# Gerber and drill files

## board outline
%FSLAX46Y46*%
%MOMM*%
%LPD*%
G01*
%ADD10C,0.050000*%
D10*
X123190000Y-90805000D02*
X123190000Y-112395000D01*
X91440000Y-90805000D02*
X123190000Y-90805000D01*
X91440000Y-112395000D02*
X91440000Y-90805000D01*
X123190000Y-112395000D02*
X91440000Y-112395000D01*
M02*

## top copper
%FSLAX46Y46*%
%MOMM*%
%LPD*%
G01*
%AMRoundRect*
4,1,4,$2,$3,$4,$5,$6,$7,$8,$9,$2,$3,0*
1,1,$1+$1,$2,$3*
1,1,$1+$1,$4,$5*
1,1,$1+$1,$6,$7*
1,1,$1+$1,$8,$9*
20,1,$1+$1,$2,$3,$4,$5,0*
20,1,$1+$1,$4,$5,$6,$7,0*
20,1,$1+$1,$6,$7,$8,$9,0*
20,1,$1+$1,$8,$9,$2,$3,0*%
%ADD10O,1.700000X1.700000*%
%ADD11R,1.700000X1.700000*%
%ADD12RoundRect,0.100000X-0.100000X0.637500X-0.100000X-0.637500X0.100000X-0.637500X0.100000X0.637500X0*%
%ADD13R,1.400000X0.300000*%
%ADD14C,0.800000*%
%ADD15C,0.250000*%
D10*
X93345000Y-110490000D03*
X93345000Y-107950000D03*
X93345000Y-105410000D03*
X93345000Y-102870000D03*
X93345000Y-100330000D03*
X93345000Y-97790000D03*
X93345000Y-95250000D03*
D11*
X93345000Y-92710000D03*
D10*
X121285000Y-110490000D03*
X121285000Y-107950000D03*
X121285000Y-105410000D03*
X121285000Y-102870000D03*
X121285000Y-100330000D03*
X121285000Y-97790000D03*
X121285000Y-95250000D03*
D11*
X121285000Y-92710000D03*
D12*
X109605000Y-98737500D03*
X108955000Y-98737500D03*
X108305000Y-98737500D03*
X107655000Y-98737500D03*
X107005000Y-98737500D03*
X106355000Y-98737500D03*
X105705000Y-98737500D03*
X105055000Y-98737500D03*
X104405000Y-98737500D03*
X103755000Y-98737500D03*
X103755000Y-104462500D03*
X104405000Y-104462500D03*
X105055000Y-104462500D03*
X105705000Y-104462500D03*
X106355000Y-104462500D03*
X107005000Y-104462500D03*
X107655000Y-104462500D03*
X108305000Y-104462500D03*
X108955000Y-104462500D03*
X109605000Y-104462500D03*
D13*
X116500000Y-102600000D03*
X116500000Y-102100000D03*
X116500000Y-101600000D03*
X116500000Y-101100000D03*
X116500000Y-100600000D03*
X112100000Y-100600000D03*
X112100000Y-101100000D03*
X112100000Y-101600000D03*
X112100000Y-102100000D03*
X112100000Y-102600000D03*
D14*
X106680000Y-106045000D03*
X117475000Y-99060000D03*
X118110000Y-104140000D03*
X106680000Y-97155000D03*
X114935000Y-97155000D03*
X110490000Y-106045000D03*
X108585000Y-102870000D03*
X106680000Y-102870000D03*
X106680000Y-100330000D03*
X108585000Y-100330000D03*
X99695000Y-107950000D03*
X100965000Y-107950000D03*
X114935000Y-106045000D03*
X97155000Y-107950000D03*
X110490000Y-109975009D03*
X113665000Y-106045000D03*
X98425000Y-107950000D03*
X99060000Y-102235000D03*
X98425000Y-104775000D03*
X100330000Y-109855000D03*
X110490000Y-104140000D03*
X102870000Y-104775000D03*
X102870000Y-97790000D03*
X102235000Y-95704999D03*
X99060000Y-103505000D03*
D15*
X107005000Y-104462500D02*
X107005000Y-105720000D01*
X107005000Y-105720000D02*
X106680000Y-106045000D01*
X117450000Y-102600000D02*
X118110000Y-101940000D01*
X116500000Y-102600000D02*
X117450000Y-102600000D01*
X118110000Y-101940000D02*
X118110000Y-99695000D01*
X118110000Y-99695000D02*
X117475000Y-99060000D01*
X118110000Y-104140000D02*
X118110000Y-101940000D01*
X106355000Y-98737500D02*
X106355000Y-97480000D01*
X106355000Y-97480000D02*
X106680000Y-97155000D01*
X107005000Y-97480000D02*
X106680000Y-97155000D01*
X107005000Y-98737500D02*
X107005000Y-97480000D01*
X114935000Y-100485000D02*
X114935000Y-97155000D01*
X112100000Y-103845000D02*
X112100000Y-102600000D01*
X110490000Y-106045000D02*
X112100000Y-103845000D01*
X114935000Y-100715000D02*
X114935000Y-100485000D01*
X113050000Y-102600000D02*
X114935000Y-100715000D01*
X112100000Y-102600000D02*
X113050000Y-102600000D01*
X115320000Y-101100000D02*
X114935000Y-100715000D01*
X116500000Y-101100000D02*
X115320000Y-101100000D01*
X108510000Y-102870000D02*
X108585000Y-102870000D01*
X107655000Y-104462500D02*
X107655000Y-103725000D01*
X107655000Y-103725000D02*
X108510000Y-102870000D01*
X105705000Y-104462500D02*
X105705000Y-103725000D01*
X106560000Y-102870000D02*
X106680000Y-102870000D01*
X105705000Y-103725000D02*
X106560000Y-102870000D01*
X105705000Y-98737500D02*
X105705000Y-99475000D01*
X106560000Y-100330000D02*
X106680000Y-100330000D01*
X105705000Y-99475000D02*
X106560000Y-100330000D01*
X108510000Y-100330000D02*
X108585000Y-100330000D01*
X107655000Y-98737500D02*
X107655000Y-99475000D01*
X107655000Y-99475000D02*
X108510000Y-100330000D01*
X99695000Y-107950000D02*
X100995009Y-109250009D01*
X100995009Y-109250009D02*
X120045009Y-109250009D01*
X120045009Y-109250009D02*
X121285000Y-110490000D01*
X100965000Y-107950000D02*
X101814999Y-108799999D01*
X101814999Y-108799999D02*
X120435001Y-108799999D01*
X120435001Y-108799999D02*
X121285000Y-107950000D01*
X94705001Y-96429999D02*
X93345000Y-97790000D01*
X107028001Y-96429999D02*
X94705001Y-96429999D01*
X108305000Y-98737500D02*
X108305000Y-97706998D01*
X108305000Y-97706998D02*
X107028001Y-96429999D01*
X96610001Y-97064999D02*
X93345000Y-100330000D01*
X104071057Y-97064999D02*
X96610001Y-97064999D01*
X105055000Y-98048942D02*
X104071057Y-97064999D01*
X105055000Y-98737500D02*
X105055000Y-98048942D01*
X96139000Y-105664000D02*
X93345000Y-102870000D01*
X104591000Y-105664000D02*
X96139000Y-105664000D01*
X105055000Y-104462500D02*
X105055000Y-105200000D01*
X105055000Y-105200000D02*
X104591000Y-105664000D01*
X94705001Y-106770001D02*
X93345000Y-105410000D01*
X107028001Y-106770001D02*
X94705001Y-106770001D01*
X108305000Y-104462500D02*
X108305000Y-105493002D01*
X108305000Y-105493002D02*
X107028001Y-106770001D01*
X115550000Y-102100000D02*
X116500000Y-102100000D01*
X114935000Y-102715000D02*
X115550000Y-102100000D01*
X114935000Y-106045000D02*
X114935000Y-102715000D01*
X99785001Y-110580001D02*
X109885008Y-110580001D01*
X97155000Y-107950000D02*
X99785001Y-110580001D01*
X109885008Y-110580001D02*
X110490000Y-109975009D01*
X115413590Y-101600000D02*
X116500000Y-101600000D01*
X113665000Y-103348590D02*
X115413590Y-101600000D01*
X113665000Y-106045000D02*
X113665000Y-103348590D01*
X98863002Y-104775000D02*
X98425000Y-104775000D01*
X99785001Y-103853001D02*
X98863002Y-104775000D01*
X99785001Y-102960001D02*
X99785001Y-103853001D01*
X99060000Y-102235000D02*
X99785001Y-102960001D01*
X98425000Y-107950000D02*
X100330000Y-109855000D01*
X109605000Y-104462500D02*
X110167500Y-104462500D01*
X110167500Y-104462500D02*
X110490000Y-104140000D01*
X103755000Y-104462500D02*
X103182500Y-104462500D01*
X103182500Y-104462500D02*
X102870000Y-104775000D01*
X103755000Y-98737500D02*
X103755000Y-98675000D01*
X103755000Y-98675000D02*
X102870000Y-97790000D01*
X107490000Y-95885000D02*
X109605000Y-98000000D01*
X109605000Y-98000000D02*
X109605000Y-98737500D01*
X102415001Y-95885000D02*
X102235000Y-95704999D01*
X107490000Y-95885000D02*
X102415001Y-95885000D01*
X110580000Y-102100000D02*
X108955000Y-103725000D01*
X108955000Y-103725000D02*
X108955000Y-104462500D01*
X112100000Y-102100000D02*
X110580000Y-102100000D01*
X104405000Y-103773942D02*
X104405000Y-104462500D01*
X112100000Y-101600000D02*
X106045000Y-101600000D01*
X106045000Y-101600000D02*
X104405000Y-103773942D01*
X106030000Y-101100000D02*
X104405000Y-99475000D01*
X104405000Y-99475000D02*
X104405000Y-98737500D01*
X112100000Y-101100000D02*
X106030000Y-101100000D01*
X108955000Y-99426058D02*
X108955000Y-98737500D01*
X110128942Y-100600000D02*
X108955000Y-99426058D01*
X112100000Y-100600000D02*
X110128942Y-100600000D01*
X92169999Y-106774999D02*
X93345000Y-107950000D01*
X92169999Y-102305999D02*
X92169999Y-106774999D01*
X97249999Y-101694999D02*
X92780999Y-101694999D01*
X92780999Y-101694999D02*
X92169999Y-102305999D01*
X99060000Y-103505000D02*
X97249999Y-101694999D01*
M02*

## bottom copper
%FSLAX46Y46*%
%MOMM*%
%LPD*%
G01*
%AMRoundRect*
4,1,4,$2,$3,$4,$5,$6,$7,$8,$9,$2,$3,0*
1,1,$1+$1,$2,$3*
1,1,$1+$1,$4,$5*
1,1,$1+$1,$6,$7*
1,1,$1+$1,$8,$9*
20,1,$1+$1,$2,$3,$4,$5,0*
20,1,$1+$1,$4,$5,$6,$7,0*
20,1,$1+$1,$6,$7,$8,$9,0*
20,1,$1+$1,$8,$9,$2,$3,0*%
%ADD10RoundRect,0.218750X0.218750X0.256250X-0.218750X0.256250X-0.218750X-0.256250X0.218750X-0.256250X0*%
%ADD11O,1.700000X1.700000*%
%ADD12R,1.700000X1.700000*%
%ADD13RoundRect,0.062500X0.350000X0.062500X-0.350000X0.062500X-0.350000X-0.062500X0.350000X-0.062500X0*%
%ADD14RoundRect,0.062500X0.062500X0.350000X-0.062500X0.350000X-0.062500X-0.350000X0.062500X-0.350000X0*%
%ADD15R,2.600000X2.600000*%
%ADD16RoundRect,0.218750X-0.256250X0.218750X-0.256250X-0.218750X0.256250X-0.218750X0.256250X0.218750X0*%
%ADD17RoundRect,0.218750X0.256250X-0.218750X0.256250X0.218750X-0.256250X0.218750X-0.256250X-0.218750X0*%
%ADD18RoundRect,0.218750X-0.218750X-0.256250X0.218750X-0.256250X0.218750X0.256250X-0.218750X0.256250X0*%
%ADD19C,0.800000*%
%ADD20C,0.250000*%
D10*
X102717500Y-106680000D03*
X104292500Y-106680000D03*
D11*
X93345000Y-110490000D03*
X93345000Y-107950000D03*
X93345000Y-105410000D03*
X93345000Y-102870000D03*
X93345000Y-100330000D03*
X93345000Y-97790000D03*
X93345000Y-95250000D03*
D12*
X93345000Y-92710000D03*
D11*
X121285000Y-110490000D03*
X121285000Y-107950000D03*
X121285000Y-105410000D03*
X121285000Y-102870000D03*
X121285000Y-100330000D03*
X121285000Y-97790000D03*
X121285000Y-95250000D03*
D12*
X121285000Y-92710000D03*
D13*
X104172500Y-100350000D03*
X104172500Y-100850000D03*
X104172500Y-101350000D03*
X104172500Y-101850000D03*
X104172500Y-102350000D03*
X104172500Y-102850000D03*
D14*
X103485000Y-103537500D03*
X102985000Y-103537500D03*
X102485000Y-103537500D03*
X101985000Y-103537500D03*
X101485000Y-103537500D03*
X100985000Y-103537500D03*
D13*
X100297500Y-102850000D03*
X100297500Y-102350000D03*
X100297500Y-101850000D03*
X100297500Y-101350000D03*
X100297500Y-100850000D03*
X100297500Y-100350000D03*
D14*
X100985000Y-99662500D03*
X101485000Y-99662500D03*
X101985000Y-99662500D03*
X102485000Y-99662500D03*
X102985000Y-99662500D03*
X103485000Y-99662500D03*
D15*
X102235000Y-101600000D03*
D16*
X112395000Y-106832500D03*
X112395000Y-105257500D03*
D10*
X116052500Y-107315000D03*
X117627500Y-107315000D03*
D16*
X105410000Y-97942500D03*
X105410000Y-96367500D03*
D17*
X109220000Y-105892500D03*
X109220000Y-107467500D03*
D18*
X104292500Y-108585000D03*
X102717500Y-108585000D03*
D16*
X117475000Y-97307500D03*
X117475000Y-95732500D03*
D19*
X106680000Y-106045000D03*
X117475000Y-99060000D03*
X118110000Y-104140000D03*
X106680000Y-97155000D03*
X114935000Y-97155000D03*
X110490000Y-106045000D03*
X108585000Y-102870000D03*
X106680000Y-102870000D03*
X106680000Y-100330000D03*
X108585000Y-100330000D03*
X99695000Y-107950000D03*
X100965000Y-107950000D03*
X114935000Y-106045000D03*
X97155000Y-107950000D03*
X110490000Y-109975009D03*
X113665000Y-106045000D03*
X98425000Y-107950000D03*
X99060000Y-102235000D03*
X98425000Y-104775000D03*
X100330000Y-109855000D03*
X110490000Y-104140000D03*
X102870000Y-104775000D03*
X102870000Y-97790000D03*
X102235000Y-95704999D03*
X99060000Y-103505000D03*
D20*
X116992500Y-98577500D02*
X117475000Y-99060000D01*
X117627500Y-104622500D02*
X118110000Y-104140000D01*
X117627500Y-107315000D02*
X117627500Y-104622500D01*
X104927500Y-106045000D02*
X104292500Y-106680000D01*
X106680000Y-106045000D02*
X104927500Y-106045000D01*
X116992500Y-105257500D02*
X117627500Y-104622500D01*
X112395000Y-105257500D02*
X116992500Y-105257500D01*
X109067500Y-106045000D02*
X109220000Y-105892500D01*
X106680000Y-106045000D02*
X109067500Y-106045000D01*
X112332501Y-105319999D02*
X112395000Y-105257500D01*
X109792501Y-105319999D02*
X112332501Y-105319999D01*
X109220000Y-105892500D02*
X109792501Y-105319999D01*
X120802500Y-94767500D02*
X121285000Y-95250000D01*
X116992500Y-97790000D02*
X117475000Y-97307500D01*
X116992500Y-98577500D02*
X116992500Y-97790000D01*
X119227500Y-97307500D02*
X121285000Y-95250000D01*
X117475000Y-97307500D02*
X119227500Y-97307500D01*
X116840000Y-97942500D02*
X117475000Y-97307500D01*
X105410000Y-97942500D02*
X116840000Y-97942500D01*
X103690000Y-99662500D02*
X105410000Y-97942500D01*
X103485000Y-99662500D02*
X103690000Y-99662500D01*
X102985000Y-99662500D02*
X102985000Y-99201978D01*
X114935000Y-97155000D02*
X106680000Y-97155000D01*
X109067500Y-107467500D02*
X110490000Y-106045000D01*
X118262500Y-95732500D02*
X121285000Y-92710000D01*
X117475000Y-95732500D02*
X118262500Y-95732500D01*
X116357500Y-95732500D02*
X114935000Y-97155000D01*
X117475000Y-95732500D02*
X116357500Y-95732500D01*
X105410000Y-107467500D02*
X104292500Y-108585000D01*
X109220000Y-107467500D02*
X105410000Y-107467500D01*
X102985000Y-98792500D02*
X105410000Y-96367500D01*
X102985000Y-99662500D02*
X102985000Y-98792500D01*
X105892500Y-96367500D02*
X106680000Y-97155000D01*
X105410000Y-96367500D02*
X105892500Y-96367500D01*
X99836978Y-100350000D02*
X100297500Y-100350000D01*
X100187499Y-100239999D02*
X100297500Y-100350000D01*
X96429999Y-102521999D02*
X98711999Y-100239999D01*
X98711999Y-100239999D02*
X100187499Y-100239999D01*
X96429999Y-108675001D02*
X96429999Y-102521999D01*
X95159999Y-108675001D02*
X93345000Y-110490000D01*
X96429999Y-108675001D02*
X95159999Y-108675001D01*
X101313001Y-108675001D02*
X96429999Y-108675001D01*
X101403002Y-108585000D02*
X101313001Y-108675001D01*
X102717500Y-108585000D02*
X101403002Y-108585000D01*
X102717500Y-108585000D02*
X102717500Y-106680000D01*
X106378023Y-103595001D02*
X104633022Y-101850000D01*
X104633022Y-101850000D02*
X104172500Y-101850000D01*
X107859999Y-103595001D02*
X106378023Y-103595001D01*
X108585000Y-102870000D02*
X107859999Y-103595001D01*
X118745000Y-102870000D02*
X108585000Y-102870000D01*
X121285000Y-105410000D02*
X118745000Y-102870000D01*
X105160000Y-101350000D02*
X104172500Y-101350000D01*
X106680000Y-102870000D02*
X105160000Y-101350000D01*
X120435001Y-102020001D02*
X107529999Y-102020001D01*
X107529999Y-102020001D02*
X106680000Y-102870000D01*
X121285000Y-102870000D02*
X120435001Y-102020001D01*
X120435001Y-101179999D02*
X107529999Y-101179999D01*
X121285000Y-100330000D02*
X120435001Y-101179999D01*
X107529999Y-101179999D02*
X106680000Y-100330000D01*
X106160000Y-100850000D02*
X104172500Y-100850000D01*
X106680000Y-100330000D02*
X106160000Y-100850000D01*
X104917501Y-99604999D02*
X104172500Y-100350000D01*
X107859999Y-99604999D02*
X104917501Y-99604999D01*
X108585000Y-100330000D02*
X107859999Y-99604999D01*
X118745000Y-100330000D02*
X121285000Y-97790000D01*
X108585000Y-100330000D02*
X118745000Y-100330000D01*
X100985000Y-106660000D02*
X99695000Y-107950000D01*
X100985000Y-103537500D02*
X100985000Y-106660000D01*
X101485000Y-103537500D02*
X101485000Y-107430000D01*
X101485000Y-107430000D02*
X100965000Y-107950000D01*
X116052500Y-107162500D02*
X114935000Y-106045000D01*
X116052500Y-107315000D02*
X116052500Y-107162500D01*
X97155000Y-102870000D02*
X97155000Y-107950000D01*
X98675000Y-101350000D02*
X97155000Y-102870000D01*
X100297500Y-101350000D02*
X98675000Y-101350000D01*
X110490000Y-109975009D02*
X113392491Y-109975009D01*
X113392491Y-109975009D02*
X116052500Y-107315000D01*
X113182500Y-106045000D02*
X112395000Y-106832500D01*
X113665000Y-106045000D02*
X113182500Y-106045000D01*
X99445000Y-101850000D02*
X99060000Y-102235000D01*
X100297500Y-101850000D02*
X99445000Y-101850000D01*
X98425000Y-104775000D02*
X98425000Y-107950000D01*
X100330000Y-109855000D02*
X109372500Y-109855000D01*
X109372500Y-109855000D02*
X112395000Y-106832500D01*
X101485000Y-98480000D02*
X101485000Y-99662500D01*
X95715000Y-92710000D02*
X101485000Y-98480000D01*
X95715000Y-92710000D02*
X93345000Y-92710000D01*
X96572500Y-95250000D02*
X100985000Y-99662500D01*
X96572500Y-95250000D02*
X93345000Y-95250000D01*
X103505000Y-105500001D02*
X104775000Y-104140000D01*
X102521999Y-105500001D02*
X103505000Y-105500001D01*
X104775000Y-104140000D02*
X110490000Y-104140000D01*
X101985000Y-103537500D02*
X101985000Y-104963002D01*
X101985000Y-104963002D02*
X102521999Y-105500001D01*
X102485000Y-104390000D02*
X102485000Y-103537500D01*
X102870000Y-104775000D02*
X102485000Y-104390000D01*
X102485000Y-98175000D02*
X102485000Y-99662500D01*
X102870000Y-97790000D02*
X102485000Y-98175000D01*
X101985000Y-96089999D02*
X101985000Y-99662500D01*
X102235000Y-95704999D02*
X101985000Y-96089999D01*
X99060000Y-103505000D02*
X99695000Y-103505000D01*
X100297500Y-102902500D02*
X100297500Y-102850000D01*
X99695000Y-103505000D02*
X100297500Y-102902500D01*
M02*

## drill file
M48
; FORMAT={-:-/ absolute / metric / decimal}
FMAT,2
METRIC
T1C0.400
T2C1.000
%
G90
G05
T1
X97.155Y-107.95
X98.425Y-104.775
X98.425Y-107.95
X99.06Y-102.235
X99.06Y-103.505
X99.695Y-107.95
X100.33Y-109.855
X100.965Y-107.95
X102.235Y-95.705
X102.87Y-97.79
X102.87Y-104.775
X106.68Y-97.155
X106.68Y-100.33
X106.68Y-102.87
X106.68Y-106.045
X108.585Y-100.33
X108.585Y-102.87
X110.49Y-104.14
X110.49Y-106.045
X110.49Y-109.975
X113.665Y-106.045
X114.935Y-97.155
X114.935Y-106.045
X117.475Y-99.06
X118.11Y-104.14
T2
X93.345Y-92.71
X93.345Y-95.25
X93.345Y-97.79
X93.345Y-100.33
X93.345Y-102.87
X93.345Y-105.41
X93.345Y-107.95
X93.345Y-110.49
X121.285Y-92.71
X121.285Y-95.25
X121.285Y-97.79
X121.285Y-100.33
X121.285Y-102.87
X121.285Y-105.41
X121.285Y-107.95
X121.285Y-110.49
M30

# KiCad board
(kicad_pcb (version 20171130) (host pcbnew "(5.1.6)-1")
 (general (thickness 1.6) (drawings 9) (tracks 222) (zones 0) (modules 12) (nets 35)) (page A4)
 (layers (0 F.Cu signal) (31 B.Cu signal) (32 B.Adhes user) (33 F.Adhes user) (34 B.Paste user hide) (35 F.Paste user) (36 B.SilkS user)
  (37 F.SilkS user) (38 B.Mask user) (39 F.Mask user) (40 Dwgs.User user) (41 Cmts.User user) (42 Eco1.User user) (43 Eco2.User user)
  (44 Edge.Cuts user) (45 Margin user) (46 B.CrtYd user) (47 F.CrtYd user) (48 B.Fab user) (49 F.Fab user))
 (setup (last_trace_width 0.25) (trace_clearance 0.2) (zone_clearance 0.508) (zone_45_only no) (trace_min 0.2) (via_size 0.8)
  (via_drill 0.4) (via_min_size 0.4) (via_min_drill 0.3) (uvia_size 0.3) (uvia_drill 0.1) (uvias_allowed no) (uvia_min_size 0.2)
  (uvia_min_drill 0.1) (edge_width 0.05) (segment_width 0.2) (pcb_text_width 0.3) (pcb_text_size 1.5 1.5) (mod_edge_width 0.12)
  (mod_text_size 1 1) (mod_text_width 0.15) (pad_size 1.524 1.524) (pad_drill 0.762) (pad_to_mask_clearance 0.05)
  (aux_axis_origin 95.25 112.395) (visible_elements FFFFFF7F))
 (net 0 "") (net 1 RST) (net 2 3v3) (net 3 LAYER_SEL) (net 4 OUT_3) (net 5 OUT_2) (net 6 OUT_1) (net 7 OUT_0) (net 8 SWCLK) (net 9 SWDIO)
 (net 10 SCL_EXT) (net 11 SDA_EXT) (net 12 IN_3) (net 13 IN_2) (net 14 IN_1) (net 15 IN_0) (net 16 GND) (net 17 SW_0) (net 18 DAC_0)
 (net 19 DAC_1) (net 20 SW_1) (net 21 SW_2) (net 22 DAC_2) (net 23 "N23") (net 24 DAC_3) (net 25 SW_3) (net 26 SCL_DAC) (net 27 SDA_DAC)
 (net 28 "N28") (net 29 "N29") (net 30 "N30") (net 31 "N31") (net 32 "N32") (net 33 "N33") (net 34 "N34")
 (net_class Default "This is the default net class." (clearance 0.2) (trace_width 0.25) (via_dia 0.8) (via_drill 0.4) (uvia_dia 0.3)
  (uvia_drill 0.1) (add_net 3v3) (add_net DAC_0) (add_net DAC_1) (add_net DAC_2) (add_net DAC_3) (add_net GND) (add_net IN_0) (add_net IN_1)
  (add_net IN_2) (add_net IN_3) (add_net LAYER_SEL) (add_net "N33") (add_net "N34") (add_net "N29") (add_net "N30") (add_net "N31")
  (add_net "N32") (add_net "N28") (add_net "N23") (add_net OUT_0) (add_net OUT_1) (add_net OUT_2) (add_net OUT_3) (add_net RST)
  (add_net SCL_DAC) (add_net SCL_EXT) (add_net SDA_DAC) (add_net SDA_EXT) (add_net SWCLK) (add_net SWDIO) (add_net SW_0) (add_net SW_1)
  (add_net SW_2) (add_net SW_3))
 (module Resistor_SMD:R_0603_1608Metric (layer B.Cu) (at 103.505 106.68 180)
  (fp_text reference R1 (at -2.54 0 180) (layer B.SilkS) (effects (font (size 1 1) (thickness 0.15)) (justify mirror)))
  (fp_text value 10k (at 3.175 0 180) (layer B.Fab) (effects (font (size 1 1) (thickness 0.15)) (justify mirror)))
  (pad 2 smd roundrect (at 0.7875 0 180) (size 0.875 0.95) (layers B.Cu B.Paste B.Mask) (roundrect_rratio 0.25) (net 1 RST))
  (pad 1 smd roundrect (at -0.7875 0 180) (size 0.875 0.95) (layers B.Cu B.Paste B.Mask) (roundrect_rratio 0.25) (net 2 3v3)))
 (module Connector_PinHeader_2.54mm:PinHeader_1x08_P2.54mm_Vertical (layer B.Cu) (at 93.345 92.71 180)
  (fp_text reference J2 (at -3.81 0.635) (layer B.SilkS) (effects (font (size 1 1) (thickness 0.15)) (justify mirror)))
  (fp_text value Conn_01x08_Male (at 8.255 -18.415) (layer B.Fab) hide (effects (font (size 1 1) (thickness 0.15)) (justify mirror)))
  (pad 8 thru_hole oval (at 0 -17.78 180) (size 1.7 1.7) (drill 1) (layers *.Cu *.Mask) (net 1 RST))
  (pad 7 thru_hole oval (at 0 -15.24 180) (size 1.7 1.7) (drill 1) (layers *.Cu *.Mask) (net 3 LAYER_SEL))
  (pad 6 thru_hole oval (at 0 -12.7 180) (size 1.7 1.7) (drill 1) (layers *.Cu *.Mask) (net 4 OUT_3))
  (pad 5 thru_hole oval (at 0 -10.16 180) (size 1.7 1.7) (drill 1) (layers *.Cu *.Mask) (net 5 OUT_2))
  (pad 4 thru_hole oval (at 0 -7.62 180) (size 1.7 1.7) (drill 1) (layers *.Cu *.Mask) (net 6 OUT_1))
  (pad 3 thru_hole oval (at 0 -5.08 180) (size 1.7 1.7) (drill 1) (layers *.Cu *.Mask) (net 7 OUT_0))
  (pad 2 thru_hole oval (at 0 -2.54 180) (size 1.7 1.7) (drill 1) (layers *.Cu *.Mask) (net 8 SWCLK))
  (pad 1 thru_hole rect (at 0 0 180) (size 1.7 1.7) (drill 1) (layers *.Cu *.Mask) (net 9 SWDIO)))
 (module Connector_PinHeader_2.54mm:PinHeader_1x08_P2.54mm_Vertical (layer B.Cu) (at 121.285 92.71 180)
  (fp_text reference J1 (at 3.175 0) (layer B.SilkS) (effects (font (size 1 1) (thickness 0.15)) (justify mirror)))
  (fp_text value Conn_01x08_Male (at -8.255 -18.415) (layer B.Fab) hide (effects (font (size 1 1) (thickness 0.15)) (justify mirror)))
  (pad 8 thru_hole oval (at 0 -17.78 180) (size 1.7 1.7) (drill 1) (layers *.Cu *.Mask) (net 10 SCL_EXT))
  (pad 7 thru_hole oval (at 0 -15.24 180) (size 1.7 1.7) (drill 1) (layers *.Cu *.Mask) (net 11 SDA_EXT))
  (pad 6 thru_hole oval (at 0 -12.7 180) (size 1.7 1.7) (drill 1) (layers *.Cu *.Mask) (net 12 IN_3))
  (pad 5 thru_hole oval (at 0 -10.16 180) (size 1.7 1.7) (drill 1) (layers *.Cu *.Mask) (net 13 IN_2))
  (pad 4 thru_hole oval (at 0 -7.62 180) (size 1.7 1.7) (drill 1) (layers *.Cu *.Mask) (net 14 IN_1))
  (pad 3 thru_hole oval (at 0 -5.08 180) (size 1.7 1.7) (drill 1) (layers *.Cu *.Mask) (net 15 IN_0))
  (pad 2 thru_hole oval (at 0 -2.54 180) (size 1.7 1.7) (drill 1) (layers *.Cu *.Mask) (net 2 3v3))
  (pad 1 thru_hole rect (at 0 0 180) (size 1.7 1.7) (drill 1) (layers *.Cu *.Mask) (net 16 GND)))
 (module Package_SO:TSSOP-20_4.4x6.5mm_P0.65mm (layer F.Cu) (at 106.68 101.6 270)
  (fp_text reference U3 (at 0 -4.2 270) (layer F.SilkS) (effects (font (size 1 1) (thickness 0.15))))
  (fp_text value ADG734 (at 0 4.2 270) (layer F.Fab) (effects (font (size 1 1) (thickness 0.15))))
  (pad 1 smd roundrect (at -2.8625 -2.925 270) (size 1.475 0.4) (layers F.Cu F.Paste F.Mask) (roundrect_rratio 0.25) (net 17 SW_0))
  (pad 2 smd roundrect (at -2.8625 -2.275 270) (size 1.475 0.4) (layers F.Cu F.Paste F.Mask) (roundrect_rratio 0.25) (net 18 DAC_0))
  (pad 3 smd roundrect (at -2.8625 -1.625 270) (size 1.475 0.4) (layers F.Cu F.Paste F.Mask) (roundrect_rratio 0.25) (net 7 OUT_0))
  (pad 4 smd roundrect (at -2.8625 -0.975 270) (size 1.475 0.4) (layers F.Cu F.Paste F.Mask) (roundrect_rratio 0.25) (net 15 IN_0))
  (pad 5 smd roundrect (at -2.8625 -0.325 270) (size 1.475 0.4) (layers F.Cu F.Paste F.Mask) (roundrect_rratio 0.25) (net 16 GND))
  (pad 6 smd roundrect (at -2.8625 0.325 270) (size 1.475 0.4) (layers F.Cu F.Paste F.Mask) (roundrect_rratio 0.25) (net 16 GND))
  (pad 7 smd roundrect (at -2.8625 0.975 270) (size 1.475 0.4) (layers F.Cu F.Paste F.Mask) (roundrect_rratio 0.25) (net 14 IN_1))
  (pad 8 smd roundrect (at -2.8625 1.625 270) (size 1.475 0.4) (layers F.Cu F.Paste F.Mask) (roundrect_rratio 0.25) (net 6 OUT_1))
  (pad 9 smd roundrect (at -2.8625 2.275 270) (size 1.475 0.4) (layers F.Cu F.Paste F.Mask) (roundrect_rratio 0.25) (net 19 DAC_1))
  (pad 10 smd roundrect (at -2.8625 2.925 270) (size 1.475 0.4) (layers F.Cu F.Paste F.Mask) (roundrect_rratio 0.25) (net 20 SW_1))
  (pad 11 smd roundrect (at 2.8625 2.925 270) (size 1.475 0.4) (layers F.Cu F.Paste F.Mask) (roundrect_rratio 0.25) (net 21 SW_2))
  (pad 12 smd roundrect (at 2.8625 2.275 270) (size 1.475 0.4) (layers F.Cu F.Paste F.Mask) (roundrect_rratio 0.25) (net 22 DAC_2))
  (pad 13 smd roundrect (at 2.8625 1.625 270) (size 1.475 0.4) (layers F.Cu F.Paste F.Mask) (roundrect_rratio 0.25) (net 5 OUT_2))
  (pad 14 smd roundrect (at 2.8625 0.975 270) (size 1.475 0.4) (layers F.Cu F.Paste F.Mask) (roundrect_rratio 0.25) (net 13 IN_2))
  (pad 15 smd roundrect (at 2.8625 0.325 270) (size 1.475 0.4) (layers F.Cu F.Paste F.Mask) (roundrect_rratio 0.25) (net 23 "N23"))
  (pad 16 smd roundrect (at 2.8625 -0.325 270) (size 1.475 0.4) (layers F.Cu F.Paste F.Mask) (roundrect_rratio 0.25) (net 2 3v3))
  (pad 17 smd roundrect (at 2.8625 -0.975 270) (size 1.475 0.4) (layers F.Cu F.Paste F.Mask) (roundrect_rratio 0.25) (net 12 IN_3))
  (pad 18 smd roundrect (at 2.8625 -1.625 270) (size 1.475 0.4) (layers F.Cu F.Paste F.Mask) (roundrect_rratio 0.25) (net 4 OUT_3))
  (pad 19 smd roundrect (at 2.8625 -2.275 270) (size 1.475 0.4) (layers F.Cu F.Paste F.Mask) (roundrect_rratio 0.25) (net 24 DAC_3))
  (pad 20 smd roundrect (at 2.8625 -2.925 270) (size 1.475 0.4) (layers F.Cu F.Paste F.Mask) (roundrect_rratio 0.25) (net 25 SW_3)))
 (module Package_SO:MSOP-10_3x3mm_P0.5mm (layer F.Cu) (at 114.3 101.6 180)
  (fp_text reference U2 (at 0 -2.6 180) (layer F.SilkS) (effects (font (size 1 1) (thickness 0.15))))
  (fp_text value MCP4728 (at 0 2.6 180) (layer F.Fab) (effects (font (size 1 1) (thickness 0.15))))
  (pad 1 smd rect (at -2.2 -1 180) (size 1.4 0.3) (layers F.Cu F.Paste F.Mask) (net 2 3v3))
  (pad 2 smd rect (at -2.2 -0.5 180) (size 1.4 0.3) (layers F.Cu F.Paste F.Mask) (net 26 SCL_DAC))
  (pad 3 smd rect (at -2.2 0 180) (size 1.4 0.3) (layers F.Cu F.Paste F.Mask) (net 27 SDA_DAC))
  (pad 4 smd rect (at -2.2 0.5 180) (size 1.4 0.3) (layers F.Cu F.Paste F.Mask) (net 16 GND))
  (pad 5 smd rect (at -2.2 1 180) (size 1.4 0.3) (layers F.Cu F.Paste F.Mask) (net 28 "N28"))
  (pad 6 smd rect (at 2.2 1 180) (size 1.4 0.3) (layers F.Cu F.Paste F.Mask) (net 18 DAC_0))
  (pad 7 smd rect (at 2.2 0.5 180) (size 1.4 0.3) (layers F.Cu F.Paste F.Mask) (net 19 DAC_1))
  (pad 8 smd rect (at 2.2 0 180) (size 1.4 0.3) (layers F.Cu F.Paste F.Mask) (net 22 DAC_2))
  (pad 9 smd rect (at 2.2 -0.5 180) (size 1.4 0.3) (layers F.Cu F.Paste F.Mask) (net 24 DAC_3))
  (pad 10 smd rect (at 2.2 -1 180) (size 1.4 0.3) (layers F.Cu F.Paste F.Mask) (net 16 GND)))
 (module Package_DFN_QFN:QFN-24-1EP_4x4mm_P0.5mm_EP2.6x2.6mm (layer B.Cu) (at 102.235 101.6 180)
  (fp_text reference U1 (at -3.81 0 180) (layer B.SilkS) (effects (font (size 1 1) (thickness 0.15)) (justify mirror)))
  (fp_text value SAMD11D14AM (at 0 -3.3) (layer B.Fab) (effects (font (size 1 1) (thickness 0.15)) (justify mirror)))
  (pad 1 smd roundrect (at -1.9375 1.25 180) (size 0.825 0.25) (layers B.Cu B.Paste B.Mask) (roundrect_rratio 0.25) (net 15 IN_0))
  (pad 2 smd roundrect (at -1.9375 0.75 180) (size 0.825 0.25) (layers B.Cu B.Paste B.Mask) (roundrect_rratio 0.25) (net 14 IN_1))
  (pad 3 smd roundrect (at -1.9375 0.25 180) (size 0.825 0.25) (layers B.Cu B.Paste B.Mask) (roundrect_rratio 0.25) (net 13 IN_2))
  (pad 4 smd roundrect (at -1.9375 -0.25 180) (size 0.825 0.25) (layers B.Cu B.Paste B.Mask) (roundrect_rratio 0.25) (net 12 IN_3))
  (pad 5 smd roundrect (at -1.9375 -0.75 180) (size 0.825 0.25) (layers B.Cu B.Paste B.Mask) (roundrect_rratio 0.25) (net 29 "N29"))
  (pad 6 smd roundrect (at -1.9375 -1.25 180) (size 0.825 0.25) (layers B.Cu B.Paste B.Mask) (roundrect_rratio 0.25) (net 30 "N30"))
  (pad 7 smd roundrect (at -1.25 -1.9375 180) (size 0.25 0.825) (layers B.Cu B.Paste B.Mask) (roundrect_rratio 0.25) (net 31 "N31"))
  (pad 8 smd roundrect (at -0.75 -1.9375 180) (size 0.25 0.825) (layers B.Cu B.Paste B.Mask) (roundrect_rratio 0.25) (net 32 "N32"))
  (pad 9 smd roundrect (at -0.25 -1.9375 180) (size 0.25 0.825) (layers B.Cu B.Paste B.Mask) (roundrect_rratio 0.25) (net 21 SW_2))
  (pad 10 smd roundrect (at 0.25 -1.9375 180) (size 0.25 0.825) (layers B.Cu B.Paste B.Mask) (roundrect_rratio 0.25) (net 25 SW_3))
  (pad 11 smd roundrect (at 0.75 -1.9375 180) (size 0.25 0.825) (layers B.Cu B.Paste B.Mask) (roundrect_rratio 0.25) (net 11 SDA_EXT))
  (pad 12 smd roundrect (at 1.25 -1.9375 180) (size 0.25 0.825) (layers B.Cu B.Paste B.Mask) (roundrect_rratio 0.25) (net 10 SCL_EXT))
  (pad 13 smd roundrect (at 1.9375 -1.25 180) (size 0.825 0.25) (layers B.Cu B.Paste B.Mask) (roundrect_rratio 0.25) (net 3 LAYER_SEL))
  (pad 14 smd roundrect (at 1.9375 -0.75 180) (size 0.825 0.25) (layers B.Cu B.Paste B.Mask) (roundrect_rratio 0.25) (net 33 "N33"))
  (pad 15 smd roundrect (at 1.9375 -0.25 180) (size 0.825 0.25) (layers B.Cu B.Paste B.Mask) (roundrect_rratio 0.25) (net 27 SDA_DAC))
  (pad 16 smd roundrect (at 1.9375 0.25 180) (size 0.825 0.25) (layers B.Cu B.Paste B.Mask) (roundrect_rratio 0.25) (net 26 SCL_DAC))
  (pad 17 smd roundrect (at 1.9375 0.75 180) (size 0.825 0.25) (layers B.Cu B.Paste B.Mask) (roundrect_rratio 0.25) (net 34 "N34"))
  (pad 18 smd roundrect (at 1.9375 1.25 180) (size 0.825 0.25) (layers B.Cu B.Paste B.Mask) (roundrect_rratio 0.25) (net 1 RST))
  (pad 19 smd roundrect (at 1.25 1.9375 180) (size 0.25 0.825) (layers B.Cu B.Paste B.Mask) (roundrect_rratio 0.25) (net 8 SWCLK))
  (pad 20 smd roundrect (at 0.75 1.9375 180) (size 0.25 0.825) (layers B.Cu B.Paste B.Mask) (roundrect_rratio 0.25) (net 9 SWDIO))
  (pad 21 smd roundrect (at 0.25 1.9375 180) (size 0.25 0.825) (layers B.Cu B.Paste B.Mask) (roundrect_rratio 0.25) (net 17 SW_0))
  (pad 22 smd roundrect (at -0.25 1.9375 180) (size 0.25 0.825) (layers B.Cu B.Paste B.Mask) (roundrect_rratio 0.25) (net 20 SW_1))
  (pad 23 smd roundrect (at -0.75 1.9375 180) (size 0.25 0.825) (layers B.Cu B.Paste B.Mask) (roundrect_rratio 0.25) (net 16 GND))
  (pad 24 smd roundrect (at -1.25 1.9375 180) (size 0.25 0.825) (layers B.Cu B.Paste B.Mask) (roundrect_rratio 0.25) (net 2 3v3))
  (pad 25 smd rect (at 0 0 180) (size 2.6 2.6) (layers B.Cu B.Mask))
  (pad "" smd roundrect (at -0.65 0.65 180) (size 1.05 1.05) (layers B.Paste) (roundrect_rratio 0.238095))
  (pad "" smd roundrect (at -0.65 -0.65 180) (size 1.05 1.05) (layers B.Paste) (roundrect_rratio 0.238095))
  (pad "" smd roundrect (at 0.65 0.65 180) (size 1.05 1.05) (layers B.Paste) (roundrect_rratio 0.238095))
  (pad "" smd roundrect (at 0.65 -0.65 180) (size 1.05 1.05) (layers B.Paste) (roundrect_rratio 0.238095)))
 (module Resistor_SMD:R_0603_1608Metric (layer B.Cu) (at 112.395 106.045 270)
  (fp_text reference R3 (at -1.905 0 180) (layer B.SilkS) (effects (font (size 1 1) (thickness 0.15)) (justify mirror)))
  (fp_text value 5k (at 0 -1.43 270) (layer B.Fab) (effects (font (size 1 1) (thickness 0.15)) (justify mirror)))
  (pad 2 smd roundrect (at 0.7875 0 270) (size 0.875 0.95) (layers B.Cu B.Paste B.Mask) (roundrect_rratio 0.25) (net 27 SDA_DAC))
  (pad 1 smd roundrect (at -0.7875 0 270) (size 0.875 0.95) (layers B.Cu B.Paste B.Mask) (roundrect_rratio 0.25) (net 2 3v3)))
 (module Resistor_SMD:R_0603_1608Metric (layer B.Cu) (at 116.84 107.315 180)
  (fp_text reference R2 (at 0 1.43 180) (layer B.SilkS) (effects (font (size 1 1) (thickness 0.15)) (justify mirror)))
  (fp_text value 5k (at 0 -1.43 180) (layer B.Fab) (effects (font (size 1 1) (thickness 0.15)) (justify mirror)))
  (pad 2 smd roundrect (at 0.7875 0 180) (size 0.875 0.95) (layers B.Cu B.Paste B.Mask) (roundrect_rratio 0.25) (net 26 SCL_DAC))
  (pad 1 smd roundrect (at -0.7875 0 180) (size 0.875 0.95) (layers B.Cu B.Paste B.Mask) (roundrect_rratio 0.25) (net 2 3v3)))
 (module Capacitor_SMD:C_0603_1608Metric (layer B.Cu) (at 105.41 97.155 270)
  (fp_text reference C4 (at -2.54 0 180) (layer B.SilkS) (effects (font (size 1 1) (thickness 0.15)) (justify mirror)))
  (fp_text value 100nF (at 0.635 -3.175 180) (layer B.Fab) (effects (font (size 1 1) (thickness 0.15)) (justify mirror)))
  (pad 2 smd roundrect (at 0.7875 0 270) (size 0.875 0.95) (layers B.Cu B.Paste B.Mask) (roundrect_rratio 0.25) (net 2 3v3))
  (pad 1 smd roundrect (at -0.7875 0 270) (size 0.875 0.95) (layers B.Cu B.Paste B.Mask) (roundrect_rratio 0.25) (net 16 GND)))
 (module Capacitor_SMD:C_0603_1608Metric (layer B.Cu) (at 109.22 106.68 90)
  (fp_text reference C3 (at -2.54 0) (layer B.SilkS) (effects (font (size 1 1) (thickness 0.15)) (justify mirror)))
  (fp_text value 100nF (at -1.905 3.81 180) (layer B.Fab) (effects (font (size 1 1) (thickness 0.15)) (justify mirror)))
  (pad 2 smd roundrect (at 0.7875 0 90) (size 0.875 0.95) (layers B.Cu B.Paste B.Mask) (roundrect_rratio 0.25) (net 2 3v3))
  (pad 1 smd roundrect (at -0.7875 0 90) (size 0.875 0.95) (layers B.Cu B.Paste B.Mask) (roundrect_rratio 0.25) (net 16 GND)))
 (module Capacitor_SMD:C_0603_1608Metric (layer B.Cu) (at 103.505 108.585)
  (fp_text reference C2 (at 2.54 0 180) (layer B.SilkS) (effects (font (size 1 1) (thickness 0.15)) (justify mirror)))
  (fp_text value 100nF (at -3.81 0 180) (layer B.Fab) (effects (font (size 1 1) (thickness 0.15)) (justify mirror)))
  (pad 2 smd roundrect (at 0.7875 0) (size 0.875 0.95) (layers B.Cu B.Paste B.Mask) (roundrect_rratio 0.25) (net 16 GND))
  (pad 1 smd roundrect (at -0.7875 0) (size 0.875 0.95) (layers B.Cu B.Paste B.Mask) (roundrect_rratio 0.25) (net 1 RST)))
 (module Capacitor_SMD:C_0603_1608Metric (layer B.Cu) (at 117.475 96.52 270)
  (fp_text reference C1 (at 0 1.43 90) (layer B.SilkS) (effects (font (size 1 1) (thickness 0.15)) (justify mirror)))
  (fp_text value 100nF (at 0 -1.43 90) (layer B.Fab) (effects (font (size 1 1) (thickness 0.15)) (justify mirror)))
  (pad 2 smd roundrect (at 0.7875 0 270) (size 0.875 0.95) (layers B.Cu B.Paste B.Mask) (roundrect_rratio 0.25) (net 2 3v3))
  (pad 1 smd roundrect (at -0.7875 0 270) (size 0.875 0.95) (layers B.Cu B.Paste B.Mask) (roundrect_rratio 0.25) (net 16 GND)))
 (gr_line (start 123.19 90.805) (end 123.19 112.395) (layer Edge.Cuts) (width 0.05))
 (gr_line (start 91.44 90.805) (end 123.19 90.805) (layer Edge.Cuts) (width 0.05))
 (gr_line (start 91.44 112.395) (end 91.44 90.805) (layer Edge.Cuts) (width 0.05))
 (gr_line (start 123.19 112.395) (end 91.44 112.395) (layer Edge.Cuts) (width 0.05))
 (via (at 106.68 106.045) (size 0.8) (drill 0.4) (layers F.Cu B.Cu) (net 2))
 (segment (start 107.005 104.4625) (end 107.005 105.72) (width 0.25) (layer F.Cu) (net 2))
 (segment (start 107.005 105.72) (end 106.68 106.045) (width 0.25) (layer F.Cu) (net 2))
 (segment (start 117.45 102.6) (end 118.11 101.94) (width 0.25) (layer F.Cu) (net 2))
 (segment (start 116.5 102.6) (end 117.45 102.6) (width 0.25) (layer F.Cu) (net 2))
 (segment (start 118.11 101.94) (end 118.11 99.695) (width 0.25) (layer F.Cu) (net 2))
 (via (at 117.475 99.06) (size 0.8) (drill 0.4) (layers F.Cu B.Cu) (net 2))
 (segment (start 118.11 99.695) (end 117.475 99.06) (width 0.25) (layer F.Cu) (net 2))
 (via (at 118.11 104.14) (size 0.8) (drill 0.4) (layers F.Cu B.Cu) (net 2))
 (segment (start 118.11 104.14) (end 118.11 101.94) (width 0.25) (layer F.Cu) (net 2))
 (segment (start 116.9925 98.5775) (end 117.475 99.06) (width 0.25) (layer B.Cu) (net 2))
 (segment (start 117.6275 104.6225) (end 118.11 104.14) (width 0.25) (layer B.Cu) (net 2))
 (segment (start 117.6275 107.315) (end 117.6275 104.6225) (width 0.25) (layer B.Cu) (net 2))
 (segment (start 104.9275 106.045) (end 104.2925 106.68) (width 0.25) (layer B.Cu) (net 2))
 (segment (start 106.68 106.045) (end 104.9275 106.045) (width 0.25) (layer B.Cu) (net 2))
 (segment (start 116.9925 105.2575) (end 117.6275 104.6225) (width 0.25) (layer B.Cu) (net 2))
 (segment (start 112.395 105.2575) (end 116.9925 105.2575) (width 0.25) (layer B.Cu) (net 2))
 (segment (start 109.0675 106.045) (end 109.22 105.8925) (width 0.25) (layer B.Cu) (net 2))
 (segment (start 106.68 106.045) (end 109.0675 106.045) (width 0.25) (layer B.Cu) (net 2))
 (segment (start 112.332501 105.319999) (end 112.395 105.2575) (width 0.25) (layer B.Cu) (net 2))
 (segment (start 109.792501 105.319999) (end 112.332501 105.319999) (width 0.25) (layer B.Cu) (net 2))
 (segment (start 109.22 105.8925) (end 109.792501 105.319999) (width 0.25) (layer B.Cu) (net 2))
 (segment (start 120.8025 94.7675) (end 121.285 95.25) (width 0.25) (layer B.Cu) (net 2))
 (segment (start 116.9925 97.79) (end 117.475 97.3075) (width 0.25) (layer B.Cu) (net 2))
 (segment (start 116.9925 98.5775) (end 116.9925 97.79) (width 0.25) (layer B.Cu) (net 2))
 (segment (start 119.2275 97.3075) (end 121.285 95.25) (width 0.25) (layer B.Cu) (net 2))
 (segment (start 117.475 97.3075) (end 119.2275 97.3075) (width 0.25) (layer B.Cu) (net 2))
 (segment (start 116.84 97.9425) (end 117.475 97.3075) (width 0.25) (layer B.Cu) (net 2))
 (segment (start 105.41 97.9425) (end 116.84 97.9425) (width 0.25) (layer B.Cu) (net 2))
 (segment (start 103.69 99.6625) (end 105.41 97.9425) (width 0.25) (layer B.Cu) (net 2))
 (segment (start 103.485 99.6625) (end 103.69 99.6625) (width 0.25) (layer B.Cu) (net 2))
 (segment (start 106.355 98.7375) (end 106.355 97.48) (width 0.25) (layer F.Cu) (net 16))
 (segment (start 106.355 97.48) (end 106.68 97.155) (width 0.25) (layer F.Cu) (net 16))
 (segment (start 107.005 97.48) (end 106.68 97.155) (width 0.25) (layer F.Cu) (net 16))
 (segment (start 107.005 98.7375) (end 107.005 97.48) (width 0.25) (layer F.Cu) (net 16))
 (via (at 106.68 97.155) (size 0.8) (drill 0.4) (layers F.Cu B.Cu) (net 16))
 (segment (start 102.985 99.6625) (end 102.985 99.201978) (width 0.25) (layer B.Cu) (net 16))
 (via (at 114.935 97.155) (size 0.8) (drill 0.4) (layers F.Cu B.Cu) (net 16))
 (segment (start 114.935 100.485) (end 114.935 97.155) (width 0.25) (layer F.Cu) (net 16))
 (segment (start 114.935 97.155) (end 106.68 97.155) (width 0.25) (layer B.Cu) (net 16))
 (segment (start 112.1 103.845) (end 112.1 102.6) (width 0.25) (layer F.Cu) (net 16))
 (via (at 110.49 106.045) (size 0.8) (drill 0.4) (layers F.Cu B.Cu) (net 16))
 (segment (start 110.49 106.045) (end 112.1 103.845) (width 0.25) (layer F.Cu) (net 16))
 (segment (start 114.935 100.715) (end 114.935 100.485) (width 0.25) (layer F.Cu) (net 16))
 (segment (start 113.05 102.6) (end 114.935 100.715) (width 0.25) (layer F.Cu) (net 16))
 (segment (start 112.1 102.6) (end 113.05 102.6) (width 0.25) (layer F.Cu) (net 16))
 (segment (start 115.32 101.1) (end 114.935 100.715) (width 0.25) (layer F.Cu) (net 16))
 (segment (start 116.5 101.1) (end 115.32 101.1) (width 0.25) (layer F.Cu) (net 16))
 (segment (start 109.0675 107.4675) (end 110.49 106.045) (width 0.25) (layer B.Cu) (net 16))
 (segment (start 118.2625 95.7325) (end 121.285 92.71) (width 0.25) (layer B.Cu) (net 16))
 (segment (start 117.475 95.7325) (end 118.2625 95.7325) (width 0.25) (layer B.Cu) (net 16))
 (segment (start 116.3575 95.7325) (end 114.935 97.155) (width 0.25) (layer B.Cu) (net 16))
 (segment (start 117.475 95.7325) (end 116.3575 95.7325) (width 0.25) (layer B.Cu) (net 16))
 (segment (start 105.41 107.4675) (end 104.2925 108.585) (width 0.25) (layer B.Cu) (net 16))
 (segment (start 109.22 107.4675) (end 105.41 107.4675) (width 0.25) (layer B.Cu) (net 16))
 (segment (start 102.985 98.7925) (end 105.41 96.3675) (width 0.25) (layer B.Cu) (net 16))
 (segment (start 102.985 99.6625) (end 102.985 98.7925) (width 0.25) (layer B.Cu) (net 16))
 (segment (start 105.8925 96.3675) (end 106.68 97.155) (width 0.25) (layer B.Cu) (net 16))
 (segment (start 105.41 96.3675) (end 105.8925 96.3675) (width 0.25) (layer B.Cu) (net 16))
 (segment (start 99.836978 100.35) (end 100.2975 100.35) (width 0.25) (layer B.Cu) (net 1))
 (segment (start 100.187499 100.239999) (end 100.2975 100.35) (width 0.25) (layer B.Cu) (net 1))
 (segment (start 96.429999 102.521999) (end 98.711999 100.239999) (width 0.25) (layer B.Cu) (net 1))
 (segment (start 98.711999 100.239999) (end 100.187499 100.239999) (width 0.25) (layer B.Cu) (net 1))
 (segment (start 96.429999 108.675001) (end 96.429999 102.521999) (width 0.25) (layer B.Cu) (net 1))
 (segment (start 95.159999 108.675001) (end 93.345 110.49) (width 0.25) (layer B.Cu) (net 1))
 (segment (start 96.429999 108.675001) (end 95.159999 108.675001) (width 0.25) (layer B.Cu) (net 1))
 (segment (start 101.313001 108.675001) (end 96.429999 108.675001) (width 0.25) (layer B.Cu) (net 1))
 (segment (start 101.403002 108.585) (end 101.313001 108.675001) (width 0.25) (layer B.Cu) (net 1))
 (segment (start 102.7175 108.585) (end 101.403002 108.585) (width 0.25) (layer B.Cu) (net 1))
 (segment (start 102.7175 108.585) (end 102.7175 106.68) (width 0.25) (layer B.Cu) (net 1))
 (via (at 108.585 102.87) (size 0.8) (drill 0.4) (layers F.Cu B.Cu) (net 12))
 (segment (start 108.51 102.87) (end 108.585 102.87) (width 0.25) (layer F.Cu) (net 12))
 (segment (start 107.655 104.4625) (end 107.655 103.725) (width 0.25) (layer F.Cu) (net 12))
 (segment (start 107.655 103.725) (end 108.51 102.87) (width 0.25) (layer F.Cu) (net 12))
 (segment (start 106.378023 103.595001) (end 104.633022 101.85) (width 0.25) (layer B.Cu) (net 12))
 (segment (start 104.633022 101.85) (end 104.1725 101.85) (width 0.25) (layer B.Cu) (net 12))
 (segment (start 107.859999 103.595001) (end 106.378023 103.595001) (width 0.25) (layer B.Cu) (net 12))
 (segment (start 108.585 102.87) (end 107.859999 103.595001) (width 0.25) (layer B.Cu) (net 12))
 (segment (start 118.745 102.87) (end 108.585 102.87) (width 0.25) (layer B.Cu) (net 12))
 (segment (start 121.285 105.41) (end 118.745 102.87) (width 0.25) (layer B.Cu) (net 12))
 (segment (start 105.705 104.4625) (end 105.705 103.725) (width 0.25) (layer F.Cu) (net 13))
 (via (at 106.68 102.87) (size 0.8) (drill 0.4) (layers F.Cu B.Cu) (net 13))
 (segment (start 106.56 102.87) (end 106.68 102.87) (width 0.25) (layer F.Cu) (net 13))
 (segment (start 105.705 103.725) (end 106.56 102.87) (width 0.25) (layer F.Cu) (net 13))
 (segment (start 105.16 101.35) (end 104.1725 101.35) (width 0.25) (layer B.Cu) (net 13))
 (segment (start 106.68 102.87) (end 105.16 101.35) (width 0.25) (layer B.Cu) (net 13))
 (segment (start 120.435001 102.020001) (end 107.529999 102.020001) (width 0.25) (layer B.Cu) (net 13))
 (segment (start 107.529999 102.020001) (end 106.68 102.87) (width 0.25) (layer B.Cu) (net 13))
 (segment (start 121.285 102.87) (end 120.435001 102.020001) (width 0.25) (layer B.Cu) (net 13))
 (via (at 106.68 100.33) (size 0.8) (drill 0.4) (layers F.Cu B.Cu) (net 14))
 (segment (start 105.705 98.7375) (end 105.705 99.475) (width 0.25) (layer F.Cu) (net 14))
 (segment (start 106.56 100.33) (end 106.68 100.33) (width 0.25) (layer F.Cu) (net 14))
 (segment (start 105.705 99.475) (end 106.56 100.33) (width 0.25) (layer F.Cu) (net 14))
 (segment (start 120.435001 101.179999) (end 107.529999 101.179999) (width 0.25) (layer B.Cu) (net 14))
 (segment (start 121.285 100.33) (end 120.435001 101.179999) (width 0.25) (layer B.Cu) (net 14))
 (segment (start 107.529999 101.179999) (end 106.68 100.33) (width 0.25) (layer B.Cu) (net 14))
 (segment (start 106.16 100.85) (end 104.1725 100.85) (width 0.25) (layer B.Cu) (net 14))
 (segment (start 106.68 100.33) (end 106.16 100.85) (width 0.25) (layer B.Cu) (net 14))
 (via (at 108.585 100.33) (size 0.8) (drill 0.4) (layers F.Cu B.Cu) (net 15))
 (segment (start 108.51 100.33) (end 108.585 100.33) (width 0.25) (layer F.Cu) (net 15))
 (segment (start 107.655 98.7375) (end 107.655 99.475) (width 0.25) (layer F.Cu) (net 15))
 (segment (start 107.655 99.475) (end 108.51 100.33) (width 0.25) (layer F.Cu) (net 15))
 (segment (start 104.917501 99.604999) (end 104.1725 100.35) (width 0.25) (layer B.Cu) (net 15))
 (segment (start 107.859999 99.604999) (end 104.917501 99.604999) (width 0.25) (layer B.Cu) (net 15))
 (segment (start 108.585 100.33) (end 107.859999 99.604999) (width 0.25) (layer B.Cu) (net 15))
 (segment (start 118.745 100.33) (end 121.285 97.79) (width 0.25) (layer B.Cu) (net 15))
 (segment (start 108.585 100.33) (end 118.745 100.33) (width 0.25) (layer B.Cu) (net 15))
 (segment (start 99.695 107.95) (end 100.995009 109.250009) (width 0.25) (layer F.Cu) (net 10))
 (segment (start 100.985 106.66) (end 99.695 107.95) (width 0.25) (layer B.Cu) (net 10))
 (segment (start 100.995009 109.250009) (end 120.045009 109.250009) (width 0.25) (layer F.Cu) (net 10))
 (via (at 99.695 107.95) (size 0.8) (drill 0.4) (layers F.Cu B.Cu) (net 10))
 (segment (start 100.985 103.5375) (end 100.985 106.66) (width 0.25) (layer B.Cu) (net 10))
 (segment (start 120.045009 109.250009) (end 121.285 110.49) (width 0.25) (layer F.Cu) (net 10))
 (segment (start 100.965 107.95) (end 101.814999 108.799999) (width 0.25) (layer F.Cu) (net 11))
 (segment (start 101.814999 108.799999) (end 120.435001 108.799999) (width 0.25) (layer F.Cu) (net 11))
 (segment (start 101.485 103.5375) (end 101.485 107.43) (width 0.25) (layer B.Cu) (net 11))
 (via (at 100.965 107.95) (size 0.8) (drill 0.4) (layers F.Cu B.Cu) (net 11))
 (segment (start 120.435001 108.799999) (end 121.285 107.95) (width 0.25) (layer F.Cu) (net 11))
 (segment (start 101.485 107.43) (end 100.965 107.95) (width 0.25) (layer B.Cu) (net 11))
 (segment (start 94.705001 96.429999) (end 93.345 97.79) (width 0.25) (layer F.Cu) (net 7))
 (segment (start 107.028001 96.429999) (end 94.705001 96.429999) (width 0.25) (layer F.Cu) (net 7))
 (segment (start 108.305 98.7375) (end 108.305 97.706998) (width 0.25) (layer F.Cu) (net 7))
 (segment (start 108.305 97.706998) (end 107.028001 96.429999) (width 0.25) (layer F.Cu) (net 7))
 (segment (start 96.610001 97.064999) (end 93.345 100.33) (width 0.25) (layer F.Cu) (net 6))
 (segment (start 104.071057 97.064999) (end 96.610001 97.064999) (width 0.25) (layer F.Cu) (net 6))
 (segment (start 105.055 98.048942) (end 104.071057 97.064999) (width 0.25) (layer F.Cu) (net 6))
 (segment (start 105.055 98.7375) (end 105.055 98.048942) (width 0.25) (layer F.Cu) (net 6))
 (segment (start 96.139 105.664) (end 93.345 102.87) (width 0.25) (layer F.Cu) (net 5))
 (segment (start 104.591 105.664) (end 96.139 105.664) (width 0.25) (layer F.Cu) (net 5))
 (segment (start 105.055 104.4625) (end 105.055 105.2) (width 0.25) (layer F.Cu) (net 5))
 (segment (start 105.055 105.2) (end 104.591 105.664) (width 0.25) (layer F.Cu) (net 5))
 (segment (start 94.705001 106.770001) (end 93.345 105.41) (width 0.25) (layer F.Cu) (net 4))
 (segment (start 107.028001 106.770001) (end 94.705001 106.770001) (width 0.25) (layer F.Cu) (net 4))
 (segment (start 108.305 104.4625) (end 108.305 105.493002) (width 0.25) (layer F.Cu) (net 4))
 (segment (start 108.305 105.493002) (end 107.028001 106.770001) (width 0.25) (layer F.Cu) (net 4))
 (segment (start 115.55 102.1) (end 116.5 102.1) (width 0.25) (layer F.Cu) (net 26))
 (via (at 114.935 106.045) (size 0.8) (drill 0.4) (layers F.Cu B.Cu) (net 26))
 (segment (start 114.935 102.715) (end 115.55 102.1) (width 0.25) (layer F.Cu) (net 26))
 (segment (start 114.935 106.045) (end 114.935 102.715) (width 0.25) (layer F.Cu) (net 26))
 (segment (start 116.0525 107.1625) (end 114.935 106.045) (width 0.25) (layer B.Cu) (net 26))
 (segment (start 116.0525 107.315) (end 116.0525 107.1625) (width 0.25) (layer B.Cu) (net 26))
 (segment (start 97.155 102.87) (end 97.155 107.95) (width 0.25) (layer B.Cu) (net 26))
 (segment (start 98.675 101.35) (end 97.155 102.87) (width 0.25) (layer B.Cu) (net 26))
 (segment (start 100.2975 101.35) (end 98.675 101.35) (width 0.25) (layer B.Cu) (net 26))
 (via (at 97.155 107.95) (size 0.8) (drill 0.4) (layers F.Cu B.Cu) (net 26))
 (segment (start 110.49 109.975009) (end 113.392491 109.975009) (width 0.25) (layer B.Cu) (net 26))
 (segment (start 113.392491 109.975009) (end 116.0525 107.315) (width 0.25) (layer B.Cu) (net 26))
 (segment (start 99.785001 110.580001) (end 109.885008 110.580001) (width 0.25) (layer F.Cu) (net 26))
 (segment (start 97.155 107.95) (end 99.785001 110.580001) (width 0.25) (layer F.Cu) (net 26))
 (via (at 110.49 109.975009) (size 0.8) (drill 0.4) (layers F.Cu B.Cu) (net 26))
 (segment (start 109.885008 110.580001) (end 110.49 109.975009) (width 0.25) (layer F.Cu) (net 26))
 (segment (start 115.41359 101.6) (end 116.5 101.6) (width 0.25) (layer F.Cu) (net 27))
 (via (at 113.665 106.045) (size 0.8) (drill 0.4) (layers F.Cu B.Cu) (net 27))
 (segment (start 113.665 103.34859) (end 115.41359 101.6) (width 0.25) (layer F.Cu) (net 27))
 (segment (start 113.665 106.045) (end 113.665 103.34859) (width 0.25) (layer F.Cu) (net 27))
 (segment (start 113.1825 106.045) (end 112.395 106.8325) (width 0.25) (layer B.Cu) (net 27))
 (segment (start 113.665 106.045) (end 113.1825 106.045) (width 0.25) (layer B.Cu) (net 27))
 (segment (start 99.445 101.85) (end 99.06 102.235) (width 0.25) (layer B.Cu) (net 27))
 (segment (start 100.2975 101.85) (end 99.445 101.85) (width 0.25) (layer B.Cu) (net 27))
 (via (at 98.425 107.95) (size 0.8) (drill 0.4) (layers F.Cu B.Cu) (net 27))
 (via (at 99.06 102.235) (size 0.8) (drill 0.4) (layers F.Cu B.Cu) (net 27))
 (via (at 98.425 104.775) (size 0.8) (drill 0.4) (layers F.Cu B.Cu) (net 27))
 (segment (start 98.425 104.775) (end 98.425 107.95) (width 0.25) (layer B.Cu) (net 27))
 (segment (start 98.863002 104.775) (end 98.425 104.775) (width 0.25) (layer F.Cu) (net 27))
 (segment (start 99.785001 103.853001) (end 98.863002 104.775) (width 0.25) (layer F.Cu) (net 27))
 (segment (start 99.785001 102.960001) (end 99.785001 103.853001) (width 0.25) (layer F.Cu) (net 27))
 (segment (start 99.06 102.235) (end 99.785001 102.960001) (width 0.25) (layer F.Cu) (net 27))
 (segment (start 100.33 109.855) (end 109.3725 109.855) (width 0.25) (layer B.Cu) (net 27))
 (via (at 100.33 109.855) (size 0.8) (drill 0.4) (layers F.Cu B.Cu) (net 27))
 (segment (start 109.3725 109.855) (end 112.395 106.8325) (width 0.25) (layer B.Cu) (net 27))
 (segment (start 98.425 107.95) (end 100.33 109.855) (width 0.25) (layer F.Cu) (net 27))
 (segment (start 101.485 98.48) (end 101.485 99.6625) (width 0.25) (layer B.Cu) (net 9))
 (segment (start 95.715 92.71) (end 101.485 98.48) (width 0.25) (layer B.Cu) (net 9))
 (segment (start 95.715 92.71) (end 93.345 92.71) (width 0.25) (layer B.Cu) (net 9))
 (segment (start 96.5725 95.25) (end 100.985 99.6625) (width 0.25) (layer B.Cu) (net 8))
 (segment (start 96.5725 95.25) (end 93.345 95.25) (width 0.25) (layer B.Cu) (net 8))
 (via (at 110.49 104.14) (size 0.8) (drill 0.4) (layers F.Cu B.Cu) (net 25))
 (segment (start 109.605 104.4625) (end 110.1675 104.4625) (width 0.25) (layer F.Cu) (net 25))
 (segment (start 110.1675 104.4625) (end 110.49 104.14) (width 0.25) (layer F.Cu) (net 25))
 (segment (start 103.505 105.500001) (end 104.775 104.14) (width 0.25) (layer B.Cu) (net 25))
 (segment (start 102.521999 105.500001) (end 103.505 105.500001) (width 0.25) (layer B.Cu) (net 25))
 (segment (start 104.775 104.14) (end 110.49 104.14) (width 0.25) (layer B.Cu) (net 25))
 (segment (start 101.985 103.5375) (end 101.985 104.963002) (width 0.25) (layer B.Cu) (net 25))
 (segment (start 101.985 104.963002) (end 102.521999 105.500001) (width 0.25) (layer B.Cu) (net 25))
 (via (at 102.87 104.775) (size 0.8) (drill 0.4) (layers F.Cu B.Cu) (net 21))
 (segment (start 103.755 104.4625) (end 103.1825 104.4625) (width 0.25) (layer F.Cu) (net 21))
 (segment (start 103.1825 104.4625) (end 102.87 104.775) (width 0.25) (layer F.Cu) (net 21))
 (segment (start 102.485 104.39) (end 102.485 103.5375) (width 0.25) (layer B.Cu) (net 21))
 (segment (start 102.87 104.775) (end 102.485 104.39) (width 0.25) (layer B.Cu) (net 21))
 (via (at 102.87 97.79) (size 0.8) (drill 0.4) (layers F.Cu B.Cu) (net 20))
 (segment (start 103.755 98.7375) (end 103.755 98.675) (width 0.25) (layer F.Cu) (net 20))
 (segment (start 103.755 98.675) (end 102.87 97.79) (width 0.25) (layer F.Cu) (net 20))
 (segment (start 102.485 98.175) (end 102.485 99.6625) (width 0.25) (layer B.Cu) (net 20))
 (segment (start 102.87 97.79) (end 102.485 98.175) (width 0.25) (layer B.Cu) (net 20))
 (segment (start 101.985 96.089999) (end 101.985 99.6625) (width 0.25) (layer B.Cu) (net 17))
 (segment (start 102.235 95.704999) (end 101.985 96.089999) (width 0.25) (layer B.Cu) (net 17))
 (via (at 102.235 95.704999) (size 0.8) (drill 0.4) (layers F.Cu B.Cu) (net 17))
 (segment (start 107.49 95.885) (end 109.605 98) (width 0.25) (layer F.Cu) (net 17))
 (segment (start 109.605 98) (end 109.605 98.7375) (width 0.25) (layer F.Cu) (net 17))
 (segment (start 102.415001 95.885) (end 102.235 95.704999) (width 0.25) (layer F.Cu) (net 17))
 (segment (start 107.49 95.885) (end 102.415001 95.885) (width 0.25) (layer F.Cu) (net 17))
 (segment (start 110.58 102.1) (end 108.955 103.725) (width 0.25) (layer F.Cu) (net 24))
 (segment (start 108.955 103.725) (end 108.955 104.4625) (width 0.25) (layer F.Cu) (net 24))
 (segment (start 112.1 102.1) (end 110.58 102.1) (width 0.25) (layer F.Cu) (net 24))
 (segment (start 104.405 103.773942) (end 104.405 104.4625) (width 0.25) (layer F.Cu) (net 22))
 (segment (start 112.1 101.6) (end 106.045 101.6) (width 0.25) (layer F.Cu) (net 22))
 (segment (start 106.045 101.6) (end 104.405 103.773942) (width 0.25) (layer F.Cu) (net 22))
 (segment (start 106.03 101.1) (end 104.405 99.475) (width 0.25) (layer F.Cu) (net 19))
 (segment (start 104.405 99.475) (end 104.405 98.7375) (width 0.25) (layer F.Cu) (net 19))
 (segment (start 112.1 101.1) (end 106.03 101.1) (width 0.25) (layer F.Cu) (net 19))
 (segment (start 108.955 99.426058) (end 108.955 98.7375) (width 0.25) (layer F.Cu) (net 18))
 (segment (start 110.128942 100.6) (end 108.955 99.426058) (width 0.25) (layer F.Cu) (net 18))
 (segment (start 112.1 100.6) (end 110.128942 100.6) (width 0.25) (layer F.Cu) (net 18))
 (via (at 99.06 103.505) (size 0.8) (drill 0.4) (layers F.Cu B.Cu) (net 3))
 (segment (start 99.06 103.505) (end 99.695 103.505) (width 0.25) (layer B.Cu) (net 3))
 (segment (start 100.2975 102.9025) (end 100.2975 102.85) (width 0.25) (layer B.Cu) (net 3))
 (segment (start 99.695 103.505) (end 100.2975 102.9025) (width 0.25) (layer B.Cu) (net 3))
 (segment (start 92.169999 106.774999) (end 93.345 107.95) (width 0.25) (layer F.Cu) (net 3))
 (segment (start 92.169999 102.305999) (end 92.169999 106.774999) (width 0.25) (layer F.Cu) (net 3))
 (segment (start 97.249999 101.694999) (end 92.780999 101.694999) (width 0.25) (layer F.Cu) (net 3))
 (segment (start 92.780999 101.694999) (end 92.169999 102.305999) (width 0.25) (layer F.Cu) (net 3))
 (segment (start 99.06 103.505) (end 97.249999 101.694999) (width 0.25) (layer F.Cu) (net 3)))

